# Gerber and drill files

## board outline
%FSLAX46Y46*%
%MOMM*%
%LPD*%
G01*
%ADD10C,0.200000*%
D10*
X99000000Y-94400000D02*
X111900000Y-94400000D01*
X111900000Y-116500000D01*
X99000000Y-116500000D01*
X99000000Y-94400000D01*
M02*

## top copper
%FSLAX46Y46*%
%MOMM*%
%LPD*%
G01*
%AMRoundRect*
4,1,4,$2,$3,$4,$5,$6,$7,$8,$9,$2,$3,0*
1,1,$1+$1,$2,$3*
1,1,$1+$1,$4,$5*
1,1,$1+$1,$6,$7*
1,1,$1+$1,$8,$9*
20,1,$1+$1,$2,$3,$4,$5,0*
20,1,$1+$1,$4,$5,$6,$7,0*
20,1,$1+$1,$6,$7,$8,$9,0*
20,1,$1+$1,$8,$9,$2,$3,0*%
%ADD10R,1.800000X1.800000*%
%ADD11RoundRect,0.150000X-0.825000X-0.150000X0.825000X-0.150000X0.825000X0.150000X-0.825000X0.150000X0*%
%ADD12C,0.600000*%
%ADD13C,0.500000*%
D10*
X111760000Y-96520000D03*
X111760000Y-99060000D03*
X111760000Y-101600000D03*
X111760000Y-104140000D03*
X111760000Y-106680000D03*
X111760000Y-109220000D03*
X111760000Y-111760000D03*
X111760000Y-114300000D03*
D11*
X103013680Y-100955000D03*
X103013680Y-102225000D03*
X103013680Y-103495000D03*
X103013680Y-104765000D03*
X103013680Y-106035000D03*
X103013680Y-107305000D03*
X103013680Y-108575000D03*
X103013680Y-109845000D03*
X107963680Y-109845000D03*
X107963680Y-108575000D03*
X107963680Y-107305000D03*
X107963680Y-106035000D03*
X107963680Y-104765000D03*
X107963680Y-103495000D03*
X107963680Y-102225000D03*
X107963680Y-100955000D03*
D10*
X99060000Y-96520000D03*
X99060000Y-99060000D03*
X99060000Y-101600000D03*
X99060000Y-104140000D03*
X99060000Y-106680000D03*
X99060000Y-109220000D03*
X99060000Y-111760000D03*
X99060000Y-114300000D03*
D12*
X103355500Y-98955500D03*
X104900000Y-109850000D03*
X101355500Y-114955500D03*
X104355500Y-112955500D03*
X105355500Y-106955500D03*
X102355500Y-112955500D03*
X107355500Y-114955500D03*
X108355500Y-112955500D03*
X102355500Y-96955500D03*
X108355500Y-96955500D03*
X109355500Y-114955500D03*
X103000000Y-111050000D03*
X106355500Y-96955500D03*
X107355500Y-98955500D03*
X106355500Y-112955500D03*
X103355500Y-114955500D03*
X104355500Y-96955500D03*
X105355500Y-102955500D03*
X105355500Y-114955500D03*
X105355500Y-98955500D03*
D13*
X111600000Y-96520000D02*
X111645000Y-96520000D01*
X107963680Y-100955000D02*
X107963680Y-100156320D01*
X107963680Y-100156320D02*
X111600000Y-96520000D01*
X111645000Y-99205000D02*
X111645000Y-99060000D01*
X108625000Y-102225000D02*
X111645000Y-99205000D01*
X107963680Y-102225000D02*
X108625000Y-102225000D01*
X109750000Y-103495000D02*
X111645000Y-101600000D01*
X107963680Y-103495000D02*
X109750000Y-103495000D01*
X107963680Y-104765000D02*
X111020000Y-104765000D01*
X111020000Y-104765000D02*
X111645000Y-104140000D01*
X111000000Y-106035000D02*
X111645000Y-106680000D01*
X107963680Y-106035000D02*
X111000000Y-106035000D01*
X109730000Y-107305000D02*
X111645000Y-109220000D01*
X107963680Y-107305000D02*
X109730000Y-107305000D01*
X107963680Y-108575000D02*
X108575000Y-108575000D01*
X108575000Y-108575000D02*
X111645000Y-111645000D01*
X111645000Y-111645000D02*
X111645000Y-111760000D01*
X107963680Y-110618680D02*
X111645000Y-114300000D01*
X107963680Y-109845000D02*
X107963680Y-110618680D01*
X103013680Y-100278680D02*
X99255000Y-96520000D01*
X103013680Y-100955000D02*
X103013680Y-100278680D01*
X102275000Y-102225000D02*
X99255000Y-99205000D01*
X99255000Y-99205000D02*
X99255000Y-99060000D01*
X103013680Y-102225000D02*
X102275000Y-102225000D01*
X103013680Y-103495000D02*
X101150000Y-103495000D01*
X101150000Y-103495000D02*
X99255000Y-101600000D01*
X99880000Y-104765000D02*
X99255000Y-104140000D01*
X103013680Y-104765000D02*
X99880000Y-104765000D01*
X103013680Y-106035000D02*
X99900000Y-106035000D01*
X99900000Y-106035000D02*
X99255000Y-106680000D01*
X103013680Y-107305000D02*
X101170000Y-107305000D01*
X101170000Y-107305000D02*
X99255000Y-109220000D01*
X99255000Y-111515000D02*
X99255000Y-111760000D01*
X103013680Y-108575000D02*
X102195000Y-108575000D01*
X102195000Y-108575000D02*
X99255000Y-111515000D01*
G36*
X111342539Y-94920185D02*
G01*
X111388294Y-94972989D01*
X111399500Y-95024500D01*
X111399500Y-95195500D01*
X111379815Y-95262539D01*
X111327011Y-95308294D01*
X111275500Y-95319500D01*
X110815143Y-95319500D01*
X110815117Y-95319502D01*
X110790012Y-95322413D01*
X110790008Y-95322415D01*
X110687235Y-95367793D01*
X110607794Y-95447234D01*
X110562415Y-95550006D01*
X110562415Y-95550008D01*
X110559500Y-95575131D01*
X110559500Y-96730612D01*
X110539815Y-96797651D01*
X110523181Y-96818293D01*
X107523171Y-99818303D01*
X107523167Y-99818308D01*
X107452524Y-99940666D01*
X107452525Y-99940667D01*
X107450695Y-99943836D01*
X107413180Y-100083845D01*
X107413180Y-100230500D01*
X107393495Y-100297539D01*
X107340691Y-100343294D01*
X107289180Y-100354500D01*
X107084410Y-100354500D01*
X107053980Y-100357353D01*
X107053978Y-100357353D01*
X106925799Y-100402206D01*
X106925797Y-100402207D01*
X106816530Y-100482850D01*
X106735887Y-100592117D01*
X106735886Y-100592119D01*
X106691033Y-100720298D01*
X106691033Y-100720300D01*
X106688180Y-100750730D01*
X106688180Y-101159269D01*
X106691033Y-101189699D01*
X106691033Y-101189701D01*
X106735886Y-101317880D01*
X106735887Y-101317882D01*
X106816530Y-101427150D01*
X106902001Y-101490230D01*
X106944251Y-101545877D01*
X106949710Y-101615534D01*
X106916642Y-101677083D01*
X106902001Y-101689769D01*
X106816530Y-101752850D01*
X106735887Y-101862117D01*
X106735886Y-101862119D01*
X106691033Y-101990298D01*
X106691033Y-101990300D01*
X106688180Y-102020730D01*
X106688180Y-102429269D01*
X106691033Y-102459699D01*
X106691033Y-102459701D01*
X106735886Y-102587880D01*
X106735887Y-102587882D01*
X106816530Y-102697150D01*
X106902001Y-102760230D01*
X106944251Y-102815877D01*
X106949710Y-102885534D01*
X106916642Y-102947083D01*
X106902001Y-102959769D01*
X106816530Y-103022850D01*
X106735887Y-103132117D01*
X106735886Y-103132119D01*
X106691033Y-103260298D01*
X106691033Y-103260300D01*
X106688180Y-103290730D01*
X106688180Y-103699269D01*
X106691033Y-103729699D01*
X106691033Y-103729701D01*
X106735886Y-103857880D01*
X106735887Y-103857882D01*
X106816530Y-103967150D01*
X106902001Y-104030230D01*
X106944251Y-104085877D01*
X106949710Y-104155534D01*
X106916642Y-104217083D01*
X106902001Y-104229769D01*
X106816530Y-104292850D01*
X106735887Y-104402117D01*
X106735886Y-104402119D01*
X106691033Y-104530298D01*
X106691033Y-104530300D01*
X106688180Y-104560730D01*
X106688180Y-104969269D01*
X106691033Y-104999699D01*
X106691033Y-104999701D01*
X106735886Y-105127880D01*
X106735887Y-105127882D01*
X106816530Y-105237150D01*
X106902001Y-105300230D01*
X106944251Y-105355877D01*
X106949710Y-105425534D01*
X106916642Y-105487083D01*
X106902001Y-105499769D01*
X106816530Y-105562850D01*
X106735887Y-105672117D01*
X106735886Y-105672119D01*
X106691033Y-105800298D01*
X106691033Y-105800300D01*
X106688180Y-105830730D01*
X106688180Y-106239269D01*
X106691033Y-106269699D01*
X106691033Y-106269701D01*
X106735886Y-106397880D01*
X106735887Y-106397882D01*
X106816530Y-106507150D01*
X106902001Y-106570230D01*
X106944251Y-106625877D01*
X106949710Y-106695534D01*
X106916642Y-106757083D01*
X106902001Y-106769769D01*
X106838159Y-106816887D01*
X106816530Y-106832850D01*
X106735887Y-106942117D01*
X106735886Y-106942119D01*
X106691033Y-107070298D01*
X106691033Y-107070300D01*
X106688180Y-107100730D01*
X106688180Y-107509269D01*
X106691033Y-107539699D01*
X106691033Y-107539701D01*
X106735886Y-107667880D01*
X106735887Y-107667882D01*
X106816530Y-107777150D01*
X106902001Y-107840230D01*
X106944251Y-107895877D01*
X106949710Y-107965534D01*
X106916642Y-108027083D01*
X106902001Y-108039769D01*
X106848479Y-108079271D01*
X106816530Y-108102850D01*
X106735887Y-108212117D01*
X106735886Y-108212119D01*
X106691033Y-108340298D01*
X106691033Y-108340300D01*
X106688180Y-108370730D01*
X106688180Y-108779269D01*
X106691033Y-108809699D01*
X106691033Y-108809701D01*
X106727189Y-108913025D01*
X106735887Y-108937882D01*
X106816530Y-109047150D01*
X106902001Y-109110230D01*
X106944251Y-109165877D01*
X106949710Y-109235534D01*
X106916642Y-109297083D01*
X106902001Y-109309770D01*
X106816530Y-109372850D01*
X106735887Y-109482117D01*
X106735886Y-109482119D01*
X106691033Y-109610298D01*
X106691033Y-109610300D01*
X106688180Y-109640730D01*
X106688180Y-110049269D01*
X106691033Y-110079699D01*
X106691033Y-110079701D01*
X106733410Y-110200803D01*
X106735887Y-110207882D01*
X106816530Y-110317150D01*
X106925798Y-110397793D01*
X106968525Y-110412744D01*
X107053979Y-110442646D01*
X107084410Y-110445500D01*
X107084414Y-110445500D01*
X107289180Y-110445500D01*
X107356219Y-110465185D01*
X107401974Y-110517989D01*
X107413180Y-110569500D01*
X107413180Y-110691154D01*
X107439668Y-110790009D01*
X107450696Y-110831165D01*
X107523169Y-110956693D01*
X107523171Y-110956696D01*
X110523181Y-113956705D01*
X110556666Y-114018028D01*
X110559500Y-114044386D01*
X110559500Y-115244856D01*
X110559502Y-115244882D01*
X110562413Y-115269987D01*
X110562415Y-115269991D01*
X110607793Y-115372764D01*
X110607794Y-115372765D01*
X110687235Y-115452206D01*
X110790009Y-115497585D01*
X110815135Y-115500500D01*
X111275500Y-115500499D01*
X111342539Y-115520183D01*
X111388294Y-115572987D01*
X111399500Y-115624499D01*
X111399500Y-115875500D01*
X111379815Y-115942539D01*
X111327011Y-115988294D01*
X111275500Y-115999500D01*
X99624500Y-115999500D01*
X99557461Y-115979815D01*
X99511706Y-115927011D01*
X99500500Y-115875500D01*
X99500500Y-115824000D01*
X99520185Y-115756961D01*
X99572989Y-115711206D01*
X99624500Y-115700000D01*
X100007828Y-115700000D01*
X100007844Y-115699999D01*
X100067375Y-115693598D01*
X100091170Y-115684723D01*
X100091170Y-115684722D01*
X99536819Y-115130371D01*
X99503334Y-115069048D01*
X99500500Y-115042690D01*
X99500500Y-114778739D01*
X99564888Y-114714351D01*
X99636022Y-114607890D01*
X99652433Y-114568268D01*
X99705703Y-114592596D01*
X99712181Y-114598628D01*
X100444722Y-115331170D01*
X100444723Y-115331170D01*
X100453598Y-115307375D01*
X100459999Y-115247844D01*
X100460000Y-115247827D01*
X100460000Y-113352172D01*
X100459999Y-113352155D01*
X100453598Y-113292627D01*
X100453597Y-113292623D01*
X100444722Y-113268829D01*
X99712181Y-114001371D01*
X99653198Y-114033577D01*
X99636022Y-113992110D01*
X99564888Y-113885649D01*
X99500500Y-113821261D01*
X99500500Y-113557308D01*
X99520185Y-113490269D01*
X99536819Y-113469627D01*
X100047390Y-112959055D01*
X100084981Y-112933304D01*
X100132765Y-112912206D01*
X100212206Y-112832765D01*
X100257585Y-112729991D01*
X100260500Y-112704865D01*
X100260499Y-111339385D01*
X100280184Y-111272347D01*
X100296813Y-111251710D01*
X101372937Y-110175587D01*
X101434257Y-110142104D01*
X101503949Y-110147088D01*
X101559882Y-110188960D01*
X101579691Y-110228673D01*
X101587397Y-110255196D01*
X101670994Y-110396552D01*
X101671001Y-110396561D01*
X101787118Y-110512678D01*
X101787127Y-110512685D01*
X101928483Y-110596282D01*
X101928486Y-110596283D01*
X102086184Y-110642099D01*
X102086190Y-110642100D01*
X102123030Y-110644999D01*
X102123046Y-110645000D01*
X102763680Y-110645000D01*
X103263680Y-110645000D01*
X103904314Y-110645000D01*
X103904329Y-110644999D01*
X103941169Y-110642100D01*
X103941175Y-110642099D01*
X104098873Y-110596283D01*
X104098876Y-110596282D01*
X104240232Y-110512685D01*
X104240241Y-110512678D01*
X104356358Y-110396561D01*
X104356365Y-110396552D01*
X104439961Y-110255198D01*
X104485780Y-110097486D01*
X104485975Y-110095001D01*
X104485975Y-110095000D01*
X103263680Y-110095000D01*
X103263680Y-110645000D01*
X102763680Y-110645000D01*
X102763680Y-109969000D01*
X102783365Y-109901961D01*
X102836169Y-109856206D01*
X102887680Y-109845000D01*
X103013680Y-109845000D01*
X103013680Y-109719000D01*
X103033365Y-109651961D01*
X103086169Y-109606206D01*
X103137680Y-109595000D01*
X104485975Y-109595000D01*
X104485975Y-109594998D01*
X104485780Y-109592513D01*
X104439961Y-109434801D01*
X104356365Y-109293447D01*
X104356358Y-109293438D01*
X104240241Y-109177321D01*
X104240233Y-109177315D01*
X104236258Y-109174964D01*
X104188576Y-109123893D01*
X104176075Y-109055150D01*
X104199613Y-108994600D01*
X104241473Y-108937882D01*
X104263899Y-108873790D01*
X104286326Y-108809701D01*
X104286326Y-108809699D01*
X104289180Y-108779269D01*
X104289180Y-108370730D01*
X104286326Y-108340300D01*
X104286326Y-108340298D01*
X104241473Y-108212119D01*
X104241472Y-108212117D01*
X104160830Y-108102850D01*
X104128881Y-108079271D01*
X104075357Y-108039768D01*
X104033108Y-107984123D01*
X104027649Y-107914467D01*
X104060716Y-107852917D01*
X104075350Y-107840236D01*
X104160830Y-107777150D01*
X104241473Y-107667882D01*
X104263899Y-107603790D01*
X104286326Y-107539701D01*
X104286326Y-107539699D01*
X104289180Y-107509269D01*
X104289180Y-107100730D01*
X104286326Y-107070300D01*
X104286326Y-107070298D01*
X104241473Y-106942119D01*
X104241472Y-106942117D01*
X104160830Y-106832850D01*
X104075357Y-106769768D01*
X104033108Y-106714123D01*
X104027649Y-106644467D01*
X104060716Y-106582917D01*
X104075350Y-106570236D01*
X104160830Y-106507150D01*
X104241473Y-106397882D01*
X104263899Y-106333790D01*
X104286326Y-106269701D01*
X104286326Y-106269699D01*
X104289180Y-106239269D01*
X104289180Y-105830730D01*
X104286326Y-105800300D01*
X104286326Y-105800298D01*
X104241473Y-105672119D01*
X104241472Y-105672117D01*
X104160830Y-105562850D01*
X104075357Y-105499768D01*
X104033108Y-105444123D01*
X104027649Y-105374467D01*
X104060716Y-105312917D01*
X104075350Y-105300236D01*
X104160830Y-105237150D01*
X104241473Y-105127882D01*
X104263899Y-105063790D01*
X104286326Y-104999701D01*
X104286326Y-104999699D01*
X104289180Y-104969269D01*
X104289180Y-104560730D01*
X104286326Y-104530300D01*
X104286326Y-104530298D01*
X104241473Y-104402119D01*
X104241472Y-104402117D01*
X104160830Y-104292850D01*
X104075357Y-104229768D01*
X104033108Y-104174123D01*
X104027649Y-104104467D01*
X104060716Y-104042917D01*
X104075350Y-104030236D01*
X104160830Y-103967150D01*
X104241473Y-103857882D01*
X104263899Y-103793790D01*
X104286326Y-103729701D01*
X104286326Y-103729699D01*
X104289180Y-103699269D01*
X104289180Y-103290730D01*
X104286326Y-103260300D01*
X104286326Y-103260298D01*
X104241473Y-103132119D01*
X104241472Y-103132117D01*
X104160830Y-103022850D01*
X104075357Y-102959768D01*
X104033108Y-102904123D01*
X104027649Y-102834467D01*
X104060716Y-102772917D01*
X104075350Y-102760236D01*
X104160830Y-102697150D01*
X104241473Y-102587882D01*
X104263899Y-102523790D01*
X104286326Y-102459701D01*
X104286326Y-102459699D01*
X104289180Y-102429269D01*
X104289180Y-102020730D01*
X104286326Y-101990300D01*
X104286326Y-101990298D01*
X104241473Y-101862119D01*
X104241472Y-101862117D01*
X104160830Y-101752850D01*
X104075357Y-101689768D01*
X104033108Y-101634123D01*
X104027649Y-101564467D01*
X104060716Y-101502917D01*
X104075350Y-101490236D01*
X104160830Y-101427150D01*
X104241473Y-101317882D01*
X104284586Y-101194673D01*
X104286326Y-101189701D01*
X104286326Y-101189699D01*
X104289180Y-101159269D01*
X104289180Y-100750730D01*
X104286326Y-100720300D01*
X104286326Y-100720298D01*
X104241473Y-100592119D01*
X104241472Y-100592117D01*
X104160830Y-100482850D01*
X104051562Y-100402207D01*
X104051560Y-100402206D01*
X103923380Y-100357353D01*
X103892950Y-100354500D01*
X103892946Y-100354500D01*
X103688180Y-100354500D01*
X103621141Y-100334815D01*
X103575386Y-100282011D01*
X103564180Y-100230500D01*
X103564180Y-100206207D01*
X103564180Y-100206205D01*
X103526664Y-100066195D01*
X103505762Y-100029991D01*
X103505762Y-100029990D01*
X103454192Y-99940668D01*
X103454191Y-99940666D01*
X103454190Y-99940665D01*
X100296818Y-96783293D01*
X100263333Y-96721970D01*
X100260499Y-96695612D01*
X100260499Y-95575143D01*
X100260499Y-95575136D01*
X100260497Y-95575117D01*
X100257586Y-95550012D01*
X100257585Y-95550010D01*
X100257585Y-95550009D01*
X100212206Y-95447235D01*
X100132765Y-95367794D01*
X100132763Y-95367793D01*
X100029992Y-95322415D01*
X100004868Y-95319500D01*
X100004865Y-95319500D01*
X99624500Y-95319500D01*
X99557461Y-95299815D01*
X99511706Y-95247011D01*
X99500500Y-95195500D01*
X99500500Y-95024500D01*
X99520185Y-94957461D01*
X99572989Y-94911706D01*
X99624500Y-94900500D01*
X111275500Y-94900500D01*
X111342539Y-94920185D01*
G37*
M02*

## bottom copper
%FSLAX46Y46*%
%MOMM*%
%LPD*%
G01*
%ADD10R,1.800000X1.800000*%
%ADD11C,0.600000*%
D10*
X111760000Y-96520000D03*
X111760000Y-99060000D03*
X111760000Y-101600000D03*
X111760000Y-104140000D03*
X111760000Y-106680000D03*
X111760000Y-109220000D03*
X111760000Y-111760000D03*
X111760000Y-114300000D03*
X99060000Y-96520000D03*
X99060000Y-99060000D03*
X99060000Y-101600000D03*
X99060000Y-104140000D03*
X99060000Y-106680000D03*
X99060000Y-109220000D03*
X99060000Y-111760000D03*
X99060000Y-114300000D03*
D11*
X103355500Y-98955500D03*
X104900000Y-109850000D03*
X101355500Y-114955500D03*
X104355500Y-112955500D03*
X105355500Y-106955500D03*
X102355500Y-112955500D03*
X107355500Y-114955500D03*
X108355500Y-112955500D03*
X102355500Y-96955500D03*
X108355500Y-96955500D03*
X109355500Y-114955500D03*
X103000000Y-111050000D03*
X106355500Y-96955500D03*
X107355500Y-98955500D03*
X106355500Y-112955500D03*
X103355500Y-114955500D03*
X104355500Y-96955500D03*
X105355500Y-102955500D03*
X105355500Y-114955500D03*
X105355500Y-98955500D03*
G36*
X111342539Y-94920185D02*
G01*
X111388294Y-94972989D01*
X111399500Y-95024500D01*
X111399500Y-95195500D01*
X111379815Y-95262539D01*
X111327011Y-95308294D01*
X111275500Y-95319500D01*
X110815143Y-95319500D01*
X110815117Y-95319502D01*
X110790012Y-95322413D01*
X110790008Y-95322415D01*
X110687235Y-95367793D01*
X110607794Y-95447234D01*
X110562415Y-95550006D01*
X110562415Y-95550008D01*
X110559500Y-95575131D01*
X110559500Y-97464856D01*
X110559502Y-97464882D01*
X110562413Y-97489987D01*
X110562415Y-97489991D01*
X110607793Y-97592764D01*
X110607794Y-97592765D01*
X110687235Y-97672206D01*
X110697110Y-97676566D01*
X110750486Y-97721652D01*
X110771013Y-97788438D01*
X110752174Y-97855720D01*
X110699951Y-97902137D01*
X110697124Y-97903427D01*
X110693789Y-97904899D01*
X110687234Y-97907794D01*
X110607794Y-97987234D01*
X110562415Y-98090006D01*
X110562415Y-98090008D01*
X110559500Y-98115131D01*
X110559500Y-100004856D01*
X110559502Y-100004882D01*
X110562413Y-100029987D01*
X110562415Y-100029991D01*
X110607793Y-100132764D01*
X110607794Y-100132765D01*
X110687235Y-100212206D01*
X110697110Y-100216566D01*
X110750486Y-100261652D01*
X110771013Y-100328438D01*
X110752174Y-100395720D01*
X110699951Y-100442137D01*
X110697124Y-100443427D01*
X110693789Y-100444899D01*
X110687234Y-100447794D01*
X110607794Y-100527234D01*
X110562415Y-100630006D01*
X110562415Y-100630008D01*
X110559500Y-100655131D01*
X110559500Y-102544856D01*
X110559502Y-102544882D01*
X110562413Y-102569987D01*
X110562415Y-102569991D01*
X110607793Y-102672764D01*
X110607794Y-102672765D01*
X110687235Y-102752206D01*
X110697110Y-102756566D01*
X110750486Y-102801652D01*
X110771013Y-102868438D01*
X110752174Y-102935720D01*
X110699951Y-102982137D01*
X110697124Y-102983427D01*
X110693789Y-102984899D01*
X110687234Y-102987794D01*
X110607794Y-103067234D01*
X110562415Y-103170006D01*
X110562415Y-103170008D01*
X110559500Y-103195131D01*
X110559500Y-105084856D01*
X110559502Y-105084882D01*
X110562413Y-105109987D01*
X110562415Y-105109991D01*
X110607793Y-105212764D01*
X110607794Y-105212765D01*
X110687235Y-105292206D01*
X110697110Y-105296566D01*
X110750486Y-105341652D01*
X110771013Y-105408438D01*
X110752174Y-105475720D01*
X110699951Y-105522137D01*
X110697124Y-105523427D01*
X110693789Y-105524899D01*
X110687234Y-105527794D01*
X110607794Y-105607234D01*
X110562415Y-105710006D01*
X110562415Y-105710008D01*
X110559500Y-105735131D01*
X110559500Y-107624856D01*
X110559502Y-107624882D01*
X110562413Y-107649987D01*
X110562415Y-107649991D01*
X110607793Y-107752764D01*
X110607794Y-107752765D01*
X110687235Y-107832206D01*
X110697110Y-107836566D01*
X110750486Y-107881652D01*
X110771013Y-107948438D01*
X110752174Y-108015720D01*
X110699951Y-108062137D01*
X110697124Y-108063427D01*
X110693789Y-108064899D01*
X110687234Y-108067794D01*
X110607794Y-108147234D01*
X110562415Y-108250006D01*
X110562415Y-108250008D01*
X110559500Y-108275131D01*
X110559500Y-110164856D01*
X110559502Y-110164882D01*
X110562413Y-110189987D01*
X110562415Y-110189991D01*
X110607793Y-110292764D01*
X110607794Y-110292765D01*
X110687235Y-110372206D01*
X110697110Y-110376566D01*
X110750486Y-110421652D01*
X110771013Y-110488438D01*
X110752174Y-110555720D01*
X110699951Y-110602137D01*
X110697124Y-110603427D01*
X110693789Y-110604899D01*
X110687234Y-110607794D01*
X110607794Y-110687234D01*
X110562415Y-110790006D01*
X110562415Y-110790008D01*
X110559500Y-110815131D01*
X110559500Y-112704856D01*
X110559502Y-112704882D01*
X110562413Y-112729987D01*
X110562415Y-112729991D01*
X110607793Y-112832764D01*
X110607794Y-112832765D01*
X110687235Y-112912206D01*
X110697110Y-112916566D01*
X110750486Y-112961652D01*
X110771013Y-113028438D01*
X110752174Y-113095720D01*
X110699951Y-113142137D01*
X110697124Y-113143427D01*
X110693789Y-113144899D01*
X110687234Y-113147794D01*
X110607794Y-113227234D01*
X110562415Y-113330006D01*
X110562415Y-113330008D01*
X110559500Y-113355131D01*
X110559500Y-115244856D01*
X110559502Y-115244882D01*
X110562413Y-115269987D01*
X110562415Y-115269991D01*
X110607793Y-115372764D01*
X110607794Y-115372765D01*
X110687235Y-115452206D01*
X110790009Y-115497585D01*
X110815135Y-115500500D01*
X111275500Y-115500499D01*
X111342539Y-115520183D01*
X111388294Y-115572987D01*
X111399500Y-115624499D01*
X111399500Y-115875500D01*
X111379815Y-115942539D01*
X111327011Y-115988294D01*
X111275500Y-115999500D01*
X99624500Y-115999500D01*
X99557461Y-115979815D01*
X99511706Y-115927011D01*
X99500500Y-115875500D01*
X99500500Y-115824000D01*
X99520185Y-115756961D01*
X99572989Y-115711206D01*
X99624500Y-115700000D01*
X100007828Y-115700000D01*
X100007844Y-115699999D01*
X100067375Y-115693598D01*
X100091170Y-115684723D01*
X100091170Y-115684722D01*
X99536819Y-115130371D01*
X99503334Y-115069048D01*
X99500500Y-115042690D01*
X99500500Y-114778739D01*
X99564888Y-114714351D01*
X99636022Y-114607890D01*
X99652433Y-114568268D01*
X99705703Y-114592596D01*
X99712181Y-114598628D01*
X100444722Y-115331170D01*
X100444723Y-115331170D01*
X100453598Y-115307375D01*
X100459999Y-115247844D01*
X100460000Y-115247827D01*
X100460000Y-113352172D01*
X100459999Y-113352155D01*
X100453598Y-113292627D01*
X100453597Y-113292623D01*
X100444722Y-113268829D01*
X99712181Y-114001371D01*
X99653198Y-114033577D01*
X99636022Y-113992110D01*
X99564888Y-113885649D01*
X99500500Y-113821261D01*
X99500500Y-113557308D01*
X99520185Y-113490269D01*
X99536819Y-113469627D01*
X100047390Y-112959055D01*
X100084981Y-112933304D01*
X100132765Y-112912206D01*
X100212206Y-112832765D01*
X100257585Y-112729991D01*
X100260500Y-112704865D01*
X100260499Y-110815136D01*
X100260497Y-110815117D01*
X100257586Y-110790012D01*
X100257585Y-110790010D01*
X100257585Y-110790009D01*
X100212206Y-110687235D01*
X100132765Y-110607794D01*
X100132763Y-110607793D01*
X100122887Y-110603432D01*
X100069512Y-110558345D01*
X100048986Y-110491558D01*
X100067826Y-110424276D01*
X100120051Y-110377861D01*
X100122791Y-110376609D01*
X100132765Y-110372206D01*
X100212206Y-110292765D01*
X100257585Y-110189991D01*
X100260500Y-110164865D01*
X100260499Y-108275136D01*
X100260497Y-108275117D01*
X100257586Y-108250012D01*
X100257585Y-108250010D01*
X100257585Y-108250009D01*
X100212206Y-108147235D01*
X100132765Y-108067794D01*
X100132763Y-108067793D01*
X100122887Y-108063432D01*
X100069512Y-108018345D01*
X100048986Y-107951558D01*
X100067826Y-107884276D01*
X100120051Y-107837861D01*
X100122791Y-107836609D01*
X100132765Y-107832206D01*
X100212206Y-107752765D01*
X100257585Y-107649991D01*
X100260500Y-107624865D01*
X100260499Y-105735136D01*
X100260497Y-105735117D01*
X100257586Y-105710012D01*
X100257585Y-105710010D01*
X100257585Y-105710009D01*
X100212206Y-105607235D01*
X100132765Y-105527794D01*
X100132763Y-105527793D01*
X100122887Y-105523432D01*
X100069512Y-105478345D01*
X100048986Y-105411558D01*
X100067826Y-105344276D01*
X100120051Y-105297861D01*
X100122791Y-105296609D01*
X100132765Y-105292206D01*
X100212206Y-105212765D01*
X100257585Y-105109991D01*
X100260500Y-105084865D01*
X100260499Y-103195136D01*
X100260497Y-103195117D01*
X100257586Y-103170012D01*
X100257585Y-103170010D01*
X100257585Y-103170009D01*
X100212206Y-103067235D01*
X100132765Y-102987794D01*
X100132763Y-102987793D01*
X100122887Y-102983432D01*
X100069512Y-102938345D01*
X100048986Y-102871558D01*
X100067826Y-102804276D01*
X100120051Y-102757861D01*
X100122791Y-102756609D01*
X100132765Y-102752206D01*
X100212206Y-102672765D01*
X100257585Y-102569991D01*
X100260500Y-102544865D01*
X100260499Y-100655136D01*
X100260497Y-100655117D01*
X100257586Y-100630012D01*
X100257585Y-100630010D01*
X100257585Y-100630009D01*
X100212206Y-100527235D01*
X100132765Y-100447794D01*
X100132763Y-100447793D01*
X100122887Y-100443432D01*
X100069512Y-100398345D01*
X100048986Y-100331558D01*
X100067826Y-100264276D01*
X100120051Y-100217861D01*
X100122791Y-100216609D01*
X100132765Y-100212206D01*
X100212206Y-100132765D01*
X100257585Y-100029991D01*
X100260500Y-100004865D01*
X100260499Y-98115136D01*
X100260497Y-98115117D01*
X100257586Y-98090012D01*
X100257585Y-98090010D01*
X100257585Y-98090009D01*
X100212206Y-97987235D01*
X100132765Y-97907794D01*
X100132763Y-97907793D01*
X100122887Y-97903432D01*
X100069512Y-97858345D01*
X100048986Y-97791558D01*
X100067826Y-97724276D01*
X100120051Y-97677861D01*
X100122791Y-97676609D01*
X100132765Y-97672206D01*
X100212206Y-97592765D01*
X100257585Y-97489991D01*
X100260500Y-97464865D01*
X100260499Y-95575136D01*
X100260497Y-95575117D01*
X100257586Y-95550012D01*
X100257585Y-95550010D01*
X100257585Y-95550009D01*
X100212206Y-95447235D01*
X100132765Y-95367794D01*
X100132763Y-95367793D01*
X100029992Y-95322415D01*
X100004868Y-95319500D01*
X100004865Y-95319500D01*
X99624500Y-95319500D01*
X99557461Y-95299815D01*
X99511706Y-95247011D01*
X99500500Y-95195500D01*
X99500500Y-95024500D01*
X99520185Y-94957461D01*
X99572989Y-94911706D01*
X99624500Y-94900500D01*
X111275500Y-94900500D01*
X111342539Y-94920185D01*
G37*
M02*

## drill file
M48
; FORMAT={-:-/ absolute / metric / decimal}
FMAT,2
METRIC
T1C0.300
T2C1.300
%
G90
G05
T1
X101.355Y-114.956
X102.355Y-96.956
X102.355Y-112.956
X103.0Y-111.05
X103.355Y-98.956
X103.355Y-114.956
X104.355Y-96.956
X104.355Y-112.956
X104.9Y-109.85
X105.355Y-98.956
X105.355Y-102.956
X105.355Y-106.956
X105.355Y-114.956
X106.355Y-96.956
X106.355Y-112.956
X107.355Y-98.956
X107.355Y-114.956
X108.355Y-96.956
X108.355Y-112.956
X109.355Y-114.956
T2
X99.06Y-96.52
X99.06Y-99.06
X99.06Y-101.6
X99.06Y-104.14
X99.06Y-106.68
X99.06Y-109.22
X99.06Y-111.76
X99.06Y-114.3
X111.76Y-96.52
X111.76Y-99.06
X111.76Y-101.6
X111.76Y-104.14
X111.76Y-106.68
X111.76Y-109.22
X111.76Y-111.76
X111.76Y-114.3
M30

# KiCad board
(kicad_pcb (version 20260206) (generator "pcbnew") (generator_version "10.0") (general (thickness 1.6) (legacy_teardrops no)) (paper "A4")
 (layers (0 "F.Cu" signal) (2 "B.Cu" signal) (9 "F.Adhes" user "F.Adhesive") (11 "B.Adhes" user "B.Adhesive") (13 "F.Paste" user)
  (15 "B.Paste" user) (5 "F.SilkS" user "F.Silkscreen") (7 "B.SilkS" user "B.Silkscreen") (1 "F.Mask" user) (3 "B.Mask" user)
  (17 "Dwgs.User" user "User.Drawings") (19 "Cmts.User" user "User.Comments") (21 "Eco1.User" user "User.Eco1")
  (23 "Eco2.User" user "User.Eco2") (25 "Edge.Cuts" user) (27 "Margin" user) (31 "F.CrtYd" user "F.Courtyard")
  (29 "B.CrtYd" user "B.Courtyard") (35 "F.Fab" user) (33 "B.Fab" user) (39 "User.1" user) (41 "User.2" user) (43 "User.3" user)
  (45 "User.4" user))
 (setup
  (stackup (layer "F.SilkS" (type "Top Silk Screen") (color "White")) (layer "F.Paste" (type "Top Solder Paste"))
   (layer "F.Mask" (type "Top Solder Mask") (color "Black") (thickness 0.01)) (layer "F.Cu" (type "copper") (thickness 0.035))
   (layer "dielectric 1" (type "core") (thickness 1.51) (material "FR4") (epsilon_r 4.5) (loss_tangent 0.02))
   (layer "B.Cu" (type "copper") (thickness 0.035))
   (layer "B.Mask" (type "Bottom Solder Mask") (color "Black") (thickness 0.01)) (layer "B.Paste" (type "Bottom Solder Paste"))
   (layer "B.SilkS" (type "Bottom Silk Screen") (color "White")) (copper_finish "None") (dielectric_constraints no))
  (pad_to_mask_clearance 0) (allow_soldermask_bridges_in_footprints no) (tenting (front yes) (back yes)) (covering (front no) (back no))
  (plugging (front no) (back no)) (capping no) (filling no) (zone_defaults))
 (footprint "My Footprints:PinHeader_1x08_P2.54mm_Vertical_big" (layer "F.Cu") (at 111.76 96.52)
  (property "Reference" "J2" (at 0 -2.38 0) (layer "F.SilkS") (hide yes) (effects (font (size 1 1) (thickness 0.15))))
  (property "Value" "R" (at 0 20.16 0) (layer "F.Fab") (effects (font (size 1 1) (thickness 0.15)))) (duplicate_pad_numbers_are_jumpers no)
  (pad "1" thru_hole rect (at 0 0) (size 1.8 1.8) (drill 1.3) (layers "*.Cu" "*.Mask") (remove_unused_layers no) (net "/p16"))
  (pad "2" thru_hole rect (at 0 2.54) (size 1.8 1.8) (drill 1.3) (layers "*.Cu" "*.Mask") (remove_unused_layers no) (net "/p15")
   (thermal_bridge_angle 45))
  (pad "3" thru_hole rect (at 0 5.08) (size 1.8 1.8) (drill 1.3) (layers "*.Cu" "*.Mask") (remove_unused_layers no) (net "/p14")
   (thermal_bridge_angle 45))
  (pad "4" thru_hole rect (at 0 7.62) (size 1.8 1.8) (drill 1.3) (layers "*.Cu" "*.Mask") (remove_unused_layers no) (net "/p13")
   (thermal_bridge_angle 45))
  (pad "5" thru_hole rect (at 0 10.16) (size 1.8 1.8) (drill 1.3) (layers "*.Cu" "*.Mask") (remove_unused_layers no) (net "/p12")
   (thermal_bridge_angle 45))
  (pad "6" thru_hole rect (at 0 12.7) (size 1.8 1.8) (drill 1.3) (layers "*.Cu" "*.Mask") (remove_unused_layers no) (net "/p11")
   (thermal_bridge_angle 45))
  (pad "7" thru_hole rect (at 0 15.24) (size 1.8 1.8) (drill 1.3) (layers "*.Cu" "*.Mask") (remove_unused_layers no) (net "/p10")
   (thermal_bridge_angle 45))
  (pad "8" thru_hole rect (at 0 17.78) (size 1.8 1.8) (drill 1.3) (layers "*.Cu" "*.Mask") (remove_unused_layers no) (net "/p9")
   (thermal_bridge_angle 45)))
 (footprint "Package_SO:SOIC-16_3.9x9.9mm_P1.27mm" (layer "F.Cu") (at 105.48868 105.4)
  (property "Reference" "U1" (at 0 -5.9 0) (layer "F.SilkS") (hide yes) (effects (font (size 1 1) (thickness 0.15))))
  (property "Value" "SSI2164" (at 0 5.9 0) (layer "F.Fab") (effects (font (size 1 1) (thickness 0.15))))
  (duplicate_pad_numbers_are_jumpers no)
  (pad "1" smd roundrect (at -2.475 -4.445) (size 1.95 0.6) (layers "F.Cu" "F.Mask" "F.Paste") (roundrect_rratio 0.25) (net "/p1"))
  (pad "2" smd roundrect (at -2.475 -3.175) (size 1.95 0.6) (layers "F.Cu" "F.Mask" "F.Paste") (roundrect_rratio 0.25) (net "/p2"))
  (pad "3" smd roundrect (at -2.475 -1.905) (size 1.95 0.6) (layers "F.Cu" "F.Mask" "F.Paste") (roundrect_rratio 0.25) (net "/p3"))
  (pad "4" smd roundrect (at -2.475 -0.635) (size 1.95 0.6) (layers "F.Cu" "F.Mask" "F.Paste") (roundrect_rratio 0.25) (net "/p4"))
  (pad "5" smd roundrect (at -2.475 0.635) (size 1.95 0.6) (layers "F.Cu" "F.Mask" "F.Paste") (roundrect_rratio 0.25) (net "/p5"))
  (pad "6" smd roundrect (at -2.475 1.905) (size 1.95 0.6) (layers "F.Cu" "F.Mask" "F.Paste") (roundrect_rratio 0.25) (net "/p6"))
  (pad "7" smd roundrect (at -2.475 3.175) (size 1.95 0.6) (layers "F.Cu" "F.Mask" "F.Paste") (roundrect_rratio 0.25) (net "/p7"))
  (pad "8" smd roundrect (at -2.475 4.445) (size 1.95 0.6) (layers "F.Cu" "F.Mask" "F.Paste") (roundrect_rratio 0.25) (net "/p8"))
  (pad "9" smd roundrect (at 2.475 4.445) (size 1.95 0.6) (layers "F.Cu" "F.Mask" "F.Paste") (roundrect_rratio 0.25) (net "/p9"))
  (pad "10" smd roundrect (at 2.475 3.175) (size 1.95 0.6) (layers "F.Cu" "F.Mask" "F.Paste") (roundrect_rratio 0.25) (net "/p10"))
  (pad "11" smd roundrect (at 2.475 1.905) (size 1.95 0.6) (layers "F.Cu" "F.Mask" "F.Paste") (roundrect_rratio 0.25) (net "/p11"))
  (pad "12" smd roundrect (at 2.475 0.635) (size 1.95 0.6) (layers "F.Cu" "F.Mask" "F.Paste") (roundrect_rratio 0.25) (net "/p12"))
  (pad "13" smd roundrect (at 2.475 -0.635) (size 1.95 0.6) (layers "F.Cu" "F.Mask" "F.Paste") (roundrect_rratio 0.25) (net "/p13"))
  (pad "14" smd roundrect (at 2.475 -1.905) (size 1.95 0.6) (layers "F.Cu" "F.Mask" "F.Paste") (roundrect_rratio 0.25) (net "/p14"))
  (pad "15" smd roundrect (at 2.475 -3.175) (size 1.95 0.6) (layers "F.Cu" "F.Mask" "F.Paste") (roundrect_rratio 0.25) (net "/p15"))
  (pad "16" smd roundrect (at 2.475 -4.445) (size 1.95 0.6) (layers "F.Cu" "F.Mask" "F.Paste") (roundrect_rratio 0.25) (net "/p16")))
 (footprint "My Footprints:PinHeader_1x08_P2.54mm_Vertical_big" (layer "F.Cu") (at 99.06 96.52)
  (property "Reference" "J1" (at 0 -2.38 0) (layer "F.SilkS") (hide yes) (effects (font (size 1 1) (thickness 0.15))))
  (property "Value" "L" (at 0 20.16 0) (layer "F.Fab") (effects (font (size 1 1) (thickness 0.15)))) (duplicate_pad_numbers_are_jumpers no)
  (pad "1" thru_hole rect (at 0 0) (size 1.8 1.8) (drill 1.3) (layers "*.Cu" "*.Mask") (remove_unused_layers no) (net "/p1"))
  (pad "2" thru_hole rect (at 0 2.54) (size 1.8 1.8) (drill 1.3) (layers "*.Cu" "*.Mask") (remove_unused_layers no) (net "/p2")
   (thermal_bridge_angle 45))
  (pad "3" thru_hole rect (at 0 5.08) (size 1.8 1.8) (drill 1.3) (layers "*.Cu" "*.Mask") (remove_unused_layers no) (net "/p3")
   (thermal_bridge_angle 45))
  (pad "4" thru_hole rect (at 0 7.62) (size 1.8 1.8) (drill 1.3) (layers "*.Cu" "*.Mask") (remove_unused_layers no) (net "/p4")
   (thermal_bridge_angle 45))
  (pad "5" thru_hole rect (at 0 10.16) (size 1.8 1.8) (drill 1.3) (layers "*.Cu" "*.Mask") (remove_unused_layers no) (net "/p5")
   (thermal_bridge_angle 45))
  (pad "6" thru_hole rect (at 0 12.7) (size 1.8 1.8) (drill 1.3) (layers "*.Cu" "*.Mask") (remove_unused_layers no) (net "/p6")
   (thermal_bridge_angle 45))
  (pad "7" thru_hole rect (at 0 15.24) (size 1.8 1.8) (drill 1.3) (layers "*.Cu" "*.Mask") (remove_unused_layers no) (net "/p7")
   (thermal_bridge_angle 45))
  (pad "8" thru_hole rect (at 0 17.78) (size 1.8 1.8) (drill 1.3) (layers "*.Cu" "*.Mask") (remove_unused_layers no) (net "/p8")
   (thermal_bridge_angle 45)))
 (gr_rect (start 99 94.4) (end 111.9 116.5) (stroke (width 0.2) (type solid)) (fill no) (layer "Edge.Cuts"))
 (segment (start 111.6 96.52) (end 111.645 96.52) (width 0.5) (layer "F.Cu") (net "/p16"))
 (segment (start 107.96368 100.955) (end 107.96368 100.15632) (width 0.5) (layer "F.Cu") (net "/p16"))
 (segment (start 107.96368 100.15632) (end 111.6 96.52) (width 0.5) (layer "F.Cu") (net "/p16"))
 (segment (start 111.645 99.205) (end 111.645 99.06) (width 0.5) (layer "F.Cu") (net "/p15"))
 (segment (start 108.625 102.225) (end 111.645 99.205) (width 0.5) (layer "F.Cu") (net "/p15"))
 (segment (start 107.96368 102.225) (end 108.625 102.225) (width 0.5) (layer "F.Cu") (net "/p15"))
 (segment (start 109.75 103.495) (end 111.645 101.6) (width 0.5) (layer "F.Cu") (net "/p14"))
 (segment (start 107.96368 103.495) (end 109.75 103.495) (width 0.5) (layer "F.Cu") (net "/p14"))
 (segment (start 107.96368 104.765) (end 111.02 104.765) (width 0.5) (layer "F.Cu") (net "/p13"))
 (segment (start 111.02 104.765) (end 111.645 104.14) (width 0.5) (layer "F.Cu") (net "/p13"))
 (segment (start 111 106.035) (end 111.645 106.68) (width 0.5) (layer "F.Cu") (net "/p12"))
 (segment (start 107.96368 106.035) (end 111 106.035) (width 0.5) (layer "F.Cu") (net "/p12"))
 (segment (start 109.73 107.305) (end 111.645 109.22) (width 0.5) (layer "F.Cu") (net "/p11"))
 (segment (start 107.96368 107.305) (end 109.73 107.305) (width 0.5) (layer "F.Cu") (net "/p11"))
 (segment (start 107.96368 108.575) (end 108.575 108.575) (width 0.5) (layer "F.Cu") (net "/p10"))
 (segment (start 108.575 108.575) (end 111.645 111.645) (width 0.5) (layer "F.Cu") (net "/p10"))
 (segment (start 111.645 111.645) (end 111.645 111.76) (width 0.5) (layer "F.Cu") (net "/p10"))
 (segment (start 107.96368 110.61868) (end 111.645 114.3) (width 0.5) (layer "F.Cu") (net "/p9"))
 (segment (start 107.96368 109.845) (end 107.96368 110.61868) (width 0.5) (layer "F.Cu") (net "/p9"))
 (segment (start 103.01368 100.27868) (end 99.255 96.52) (width 0.5) (layer "F.Cu") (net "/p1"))
 (segment (start 103.01368 100.955) (end 103.01368 100.27868) (width 0.5) (layer "F.Cu") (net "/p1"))
 (segment (start 102.275 102.225) (end 99.255 99.205) (width 0.5) (layer "F.Cu") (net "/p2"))
 (segment (start 99.255 99.205) (end 99.255 99.06) (width 0.5) (layer "F.Cu") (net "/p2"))
 (segment (start 103.01368 102.225) (end 102.275 102.225) (width 0.5) (layer "F.Cu") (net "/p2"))
 (segment (start 103.01368 103.495) (end 101.15 103.495) (width 0.5) (layer "F.Cu") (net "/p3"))
 (segment (start 101.15 103.495) (end 99.255 101.6) (width 0.5) (layer "F.Cu") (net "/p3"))
 (segment (start 99.88 104.765) (end 99.255 104.14) (width 0.5) (layer "F.Cu") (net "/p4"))
 (segment (start 103.01368 104.765) (end 99.88 104.765) (width 0.5) (layer "F.Cu") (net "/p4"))
 (segment (start 103.01368 106.035) (end 99.9 106.035) (width 0.5) (layer "F.Cu") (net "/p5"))
 (segment (start 99.9 106.035) (end 99.255 106.68) (width 0.5) (layer "F.Cu") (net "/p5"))
 (segment (start 103.01368 107.305) (end 101.17 107.305) (width 0.5) (layer "F.Cu") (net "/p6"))
 (segment (start 101.17 107.305) (end 99.255 109.22) (width 0.5) (layer "F.Cu") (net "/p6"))
 (segment (start 99.255 111.515) (end 99.255 111.76) (width 0.5) (layer "F.Cu") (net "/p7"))
 (segment (start 103.01368 108.575) (end 102.195 108.575) (width 0.5) (layer "F.Cu") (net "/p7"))
 (segment (start 102.195 108.575) (end 99.255 111.515) (width 0.5) (layer "F.Cu") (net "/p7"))
 (via (at 103.3555 98.9555) (size 0.6) (drill 0.3) (layers "F.Cu" "B.Cu") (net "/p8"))
 (via (at 104.9 109.85) (size 0.6) (drill 0.3) (layers "F.Cu" "B.Cu") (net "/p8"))
 (via (at 101.3555 114.9555) (size 0.6) (drill 0.3) (layers "F.Cu" "B.Cu") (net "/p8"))
 (via (at 104.3555 112.9555) (size 0.6) (drill 0.3) (layers "F.Cu" "B.Cu") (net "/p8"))
 (via (at 105.3555 106.9555) (size 0.6) (drill 0.3) (layers "F.Cu" "B.Cu") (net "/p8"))
 (via (at 102.3555 112.9555) (size 0.6) (drill 0.3) (layers "F.Cu" "B.Cu") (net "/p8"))
 (via (at 107.3555 114.9555) (size 0.6) (drill 0.3) (layers "F.Cu" "B.Cu") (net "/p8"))
 (via (at 108.3555 112.9555) (size 0.6) (drill 0.3) (layers "F.Cu" "B.Cu") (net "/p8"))
 (via (at 102.3555 96.9555) (size 0.6) (drill 0.3) (layers "F.Cu" "B.Cu") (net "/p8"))
 (via (at 108.3555 96.9555) (size 0.6) (drill 0.3) (layers "F.Cu" "B.Cu") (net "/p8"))
 (via (at 109.3555 114.9555) (size 0.6) (drill 0.3) (layers "F.Cu" "B.Cu") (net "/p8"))
 (via (at 103 111.05) (size 0.6) (drill 0.3) (layers "F.Cu" "B.Cu") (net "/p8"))
 (via (at 106.3555 96.9555) (size 0.6) (drill 0.3) (layers "F.Cu" "B.Cu") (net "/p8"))
 (via (at 107.3555 98.9555) (size 0.6) (drill 0.3) (layers "F.Cu" "B.Cu") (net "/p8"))
 (via (at 106.3555 112.9555) (size 0.6) (drill 0.3) (layers "F.Cu" "B.Cu") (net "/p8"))
 (via (at 103.3555 114.9555) (size 0.6) (drill 0.3) (layers "F.Cu" "B.Cu") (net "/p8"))
 (via (at 104.3555 96.9555) (size 0.6) (drill 0.3) (layers "F.Cu" "B.Cu") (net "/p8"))
 (via (at 105.3555 102.9555) (size 0.6) (drill 0.3) (layers "F.Cu" "B.Cu") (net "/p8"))
 (via (at 105.3555 114.9555) (size 0.6) (drill 0.3) (layers "F.Cu" "B.Cu") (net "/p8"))
 (via (at 105.3555 98.9555) (size 0.6) (drill 0.3) (layers "F.Cu" "B.Cu") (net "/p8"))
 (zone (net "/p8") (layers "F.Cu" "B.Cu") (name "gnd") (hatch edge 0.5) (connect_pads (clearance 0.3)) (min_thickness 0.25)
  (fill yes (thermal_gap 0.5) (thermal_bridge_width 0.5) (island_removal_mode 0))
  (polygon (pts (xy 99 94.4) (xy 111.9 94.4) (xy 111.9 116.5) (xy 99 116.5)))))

